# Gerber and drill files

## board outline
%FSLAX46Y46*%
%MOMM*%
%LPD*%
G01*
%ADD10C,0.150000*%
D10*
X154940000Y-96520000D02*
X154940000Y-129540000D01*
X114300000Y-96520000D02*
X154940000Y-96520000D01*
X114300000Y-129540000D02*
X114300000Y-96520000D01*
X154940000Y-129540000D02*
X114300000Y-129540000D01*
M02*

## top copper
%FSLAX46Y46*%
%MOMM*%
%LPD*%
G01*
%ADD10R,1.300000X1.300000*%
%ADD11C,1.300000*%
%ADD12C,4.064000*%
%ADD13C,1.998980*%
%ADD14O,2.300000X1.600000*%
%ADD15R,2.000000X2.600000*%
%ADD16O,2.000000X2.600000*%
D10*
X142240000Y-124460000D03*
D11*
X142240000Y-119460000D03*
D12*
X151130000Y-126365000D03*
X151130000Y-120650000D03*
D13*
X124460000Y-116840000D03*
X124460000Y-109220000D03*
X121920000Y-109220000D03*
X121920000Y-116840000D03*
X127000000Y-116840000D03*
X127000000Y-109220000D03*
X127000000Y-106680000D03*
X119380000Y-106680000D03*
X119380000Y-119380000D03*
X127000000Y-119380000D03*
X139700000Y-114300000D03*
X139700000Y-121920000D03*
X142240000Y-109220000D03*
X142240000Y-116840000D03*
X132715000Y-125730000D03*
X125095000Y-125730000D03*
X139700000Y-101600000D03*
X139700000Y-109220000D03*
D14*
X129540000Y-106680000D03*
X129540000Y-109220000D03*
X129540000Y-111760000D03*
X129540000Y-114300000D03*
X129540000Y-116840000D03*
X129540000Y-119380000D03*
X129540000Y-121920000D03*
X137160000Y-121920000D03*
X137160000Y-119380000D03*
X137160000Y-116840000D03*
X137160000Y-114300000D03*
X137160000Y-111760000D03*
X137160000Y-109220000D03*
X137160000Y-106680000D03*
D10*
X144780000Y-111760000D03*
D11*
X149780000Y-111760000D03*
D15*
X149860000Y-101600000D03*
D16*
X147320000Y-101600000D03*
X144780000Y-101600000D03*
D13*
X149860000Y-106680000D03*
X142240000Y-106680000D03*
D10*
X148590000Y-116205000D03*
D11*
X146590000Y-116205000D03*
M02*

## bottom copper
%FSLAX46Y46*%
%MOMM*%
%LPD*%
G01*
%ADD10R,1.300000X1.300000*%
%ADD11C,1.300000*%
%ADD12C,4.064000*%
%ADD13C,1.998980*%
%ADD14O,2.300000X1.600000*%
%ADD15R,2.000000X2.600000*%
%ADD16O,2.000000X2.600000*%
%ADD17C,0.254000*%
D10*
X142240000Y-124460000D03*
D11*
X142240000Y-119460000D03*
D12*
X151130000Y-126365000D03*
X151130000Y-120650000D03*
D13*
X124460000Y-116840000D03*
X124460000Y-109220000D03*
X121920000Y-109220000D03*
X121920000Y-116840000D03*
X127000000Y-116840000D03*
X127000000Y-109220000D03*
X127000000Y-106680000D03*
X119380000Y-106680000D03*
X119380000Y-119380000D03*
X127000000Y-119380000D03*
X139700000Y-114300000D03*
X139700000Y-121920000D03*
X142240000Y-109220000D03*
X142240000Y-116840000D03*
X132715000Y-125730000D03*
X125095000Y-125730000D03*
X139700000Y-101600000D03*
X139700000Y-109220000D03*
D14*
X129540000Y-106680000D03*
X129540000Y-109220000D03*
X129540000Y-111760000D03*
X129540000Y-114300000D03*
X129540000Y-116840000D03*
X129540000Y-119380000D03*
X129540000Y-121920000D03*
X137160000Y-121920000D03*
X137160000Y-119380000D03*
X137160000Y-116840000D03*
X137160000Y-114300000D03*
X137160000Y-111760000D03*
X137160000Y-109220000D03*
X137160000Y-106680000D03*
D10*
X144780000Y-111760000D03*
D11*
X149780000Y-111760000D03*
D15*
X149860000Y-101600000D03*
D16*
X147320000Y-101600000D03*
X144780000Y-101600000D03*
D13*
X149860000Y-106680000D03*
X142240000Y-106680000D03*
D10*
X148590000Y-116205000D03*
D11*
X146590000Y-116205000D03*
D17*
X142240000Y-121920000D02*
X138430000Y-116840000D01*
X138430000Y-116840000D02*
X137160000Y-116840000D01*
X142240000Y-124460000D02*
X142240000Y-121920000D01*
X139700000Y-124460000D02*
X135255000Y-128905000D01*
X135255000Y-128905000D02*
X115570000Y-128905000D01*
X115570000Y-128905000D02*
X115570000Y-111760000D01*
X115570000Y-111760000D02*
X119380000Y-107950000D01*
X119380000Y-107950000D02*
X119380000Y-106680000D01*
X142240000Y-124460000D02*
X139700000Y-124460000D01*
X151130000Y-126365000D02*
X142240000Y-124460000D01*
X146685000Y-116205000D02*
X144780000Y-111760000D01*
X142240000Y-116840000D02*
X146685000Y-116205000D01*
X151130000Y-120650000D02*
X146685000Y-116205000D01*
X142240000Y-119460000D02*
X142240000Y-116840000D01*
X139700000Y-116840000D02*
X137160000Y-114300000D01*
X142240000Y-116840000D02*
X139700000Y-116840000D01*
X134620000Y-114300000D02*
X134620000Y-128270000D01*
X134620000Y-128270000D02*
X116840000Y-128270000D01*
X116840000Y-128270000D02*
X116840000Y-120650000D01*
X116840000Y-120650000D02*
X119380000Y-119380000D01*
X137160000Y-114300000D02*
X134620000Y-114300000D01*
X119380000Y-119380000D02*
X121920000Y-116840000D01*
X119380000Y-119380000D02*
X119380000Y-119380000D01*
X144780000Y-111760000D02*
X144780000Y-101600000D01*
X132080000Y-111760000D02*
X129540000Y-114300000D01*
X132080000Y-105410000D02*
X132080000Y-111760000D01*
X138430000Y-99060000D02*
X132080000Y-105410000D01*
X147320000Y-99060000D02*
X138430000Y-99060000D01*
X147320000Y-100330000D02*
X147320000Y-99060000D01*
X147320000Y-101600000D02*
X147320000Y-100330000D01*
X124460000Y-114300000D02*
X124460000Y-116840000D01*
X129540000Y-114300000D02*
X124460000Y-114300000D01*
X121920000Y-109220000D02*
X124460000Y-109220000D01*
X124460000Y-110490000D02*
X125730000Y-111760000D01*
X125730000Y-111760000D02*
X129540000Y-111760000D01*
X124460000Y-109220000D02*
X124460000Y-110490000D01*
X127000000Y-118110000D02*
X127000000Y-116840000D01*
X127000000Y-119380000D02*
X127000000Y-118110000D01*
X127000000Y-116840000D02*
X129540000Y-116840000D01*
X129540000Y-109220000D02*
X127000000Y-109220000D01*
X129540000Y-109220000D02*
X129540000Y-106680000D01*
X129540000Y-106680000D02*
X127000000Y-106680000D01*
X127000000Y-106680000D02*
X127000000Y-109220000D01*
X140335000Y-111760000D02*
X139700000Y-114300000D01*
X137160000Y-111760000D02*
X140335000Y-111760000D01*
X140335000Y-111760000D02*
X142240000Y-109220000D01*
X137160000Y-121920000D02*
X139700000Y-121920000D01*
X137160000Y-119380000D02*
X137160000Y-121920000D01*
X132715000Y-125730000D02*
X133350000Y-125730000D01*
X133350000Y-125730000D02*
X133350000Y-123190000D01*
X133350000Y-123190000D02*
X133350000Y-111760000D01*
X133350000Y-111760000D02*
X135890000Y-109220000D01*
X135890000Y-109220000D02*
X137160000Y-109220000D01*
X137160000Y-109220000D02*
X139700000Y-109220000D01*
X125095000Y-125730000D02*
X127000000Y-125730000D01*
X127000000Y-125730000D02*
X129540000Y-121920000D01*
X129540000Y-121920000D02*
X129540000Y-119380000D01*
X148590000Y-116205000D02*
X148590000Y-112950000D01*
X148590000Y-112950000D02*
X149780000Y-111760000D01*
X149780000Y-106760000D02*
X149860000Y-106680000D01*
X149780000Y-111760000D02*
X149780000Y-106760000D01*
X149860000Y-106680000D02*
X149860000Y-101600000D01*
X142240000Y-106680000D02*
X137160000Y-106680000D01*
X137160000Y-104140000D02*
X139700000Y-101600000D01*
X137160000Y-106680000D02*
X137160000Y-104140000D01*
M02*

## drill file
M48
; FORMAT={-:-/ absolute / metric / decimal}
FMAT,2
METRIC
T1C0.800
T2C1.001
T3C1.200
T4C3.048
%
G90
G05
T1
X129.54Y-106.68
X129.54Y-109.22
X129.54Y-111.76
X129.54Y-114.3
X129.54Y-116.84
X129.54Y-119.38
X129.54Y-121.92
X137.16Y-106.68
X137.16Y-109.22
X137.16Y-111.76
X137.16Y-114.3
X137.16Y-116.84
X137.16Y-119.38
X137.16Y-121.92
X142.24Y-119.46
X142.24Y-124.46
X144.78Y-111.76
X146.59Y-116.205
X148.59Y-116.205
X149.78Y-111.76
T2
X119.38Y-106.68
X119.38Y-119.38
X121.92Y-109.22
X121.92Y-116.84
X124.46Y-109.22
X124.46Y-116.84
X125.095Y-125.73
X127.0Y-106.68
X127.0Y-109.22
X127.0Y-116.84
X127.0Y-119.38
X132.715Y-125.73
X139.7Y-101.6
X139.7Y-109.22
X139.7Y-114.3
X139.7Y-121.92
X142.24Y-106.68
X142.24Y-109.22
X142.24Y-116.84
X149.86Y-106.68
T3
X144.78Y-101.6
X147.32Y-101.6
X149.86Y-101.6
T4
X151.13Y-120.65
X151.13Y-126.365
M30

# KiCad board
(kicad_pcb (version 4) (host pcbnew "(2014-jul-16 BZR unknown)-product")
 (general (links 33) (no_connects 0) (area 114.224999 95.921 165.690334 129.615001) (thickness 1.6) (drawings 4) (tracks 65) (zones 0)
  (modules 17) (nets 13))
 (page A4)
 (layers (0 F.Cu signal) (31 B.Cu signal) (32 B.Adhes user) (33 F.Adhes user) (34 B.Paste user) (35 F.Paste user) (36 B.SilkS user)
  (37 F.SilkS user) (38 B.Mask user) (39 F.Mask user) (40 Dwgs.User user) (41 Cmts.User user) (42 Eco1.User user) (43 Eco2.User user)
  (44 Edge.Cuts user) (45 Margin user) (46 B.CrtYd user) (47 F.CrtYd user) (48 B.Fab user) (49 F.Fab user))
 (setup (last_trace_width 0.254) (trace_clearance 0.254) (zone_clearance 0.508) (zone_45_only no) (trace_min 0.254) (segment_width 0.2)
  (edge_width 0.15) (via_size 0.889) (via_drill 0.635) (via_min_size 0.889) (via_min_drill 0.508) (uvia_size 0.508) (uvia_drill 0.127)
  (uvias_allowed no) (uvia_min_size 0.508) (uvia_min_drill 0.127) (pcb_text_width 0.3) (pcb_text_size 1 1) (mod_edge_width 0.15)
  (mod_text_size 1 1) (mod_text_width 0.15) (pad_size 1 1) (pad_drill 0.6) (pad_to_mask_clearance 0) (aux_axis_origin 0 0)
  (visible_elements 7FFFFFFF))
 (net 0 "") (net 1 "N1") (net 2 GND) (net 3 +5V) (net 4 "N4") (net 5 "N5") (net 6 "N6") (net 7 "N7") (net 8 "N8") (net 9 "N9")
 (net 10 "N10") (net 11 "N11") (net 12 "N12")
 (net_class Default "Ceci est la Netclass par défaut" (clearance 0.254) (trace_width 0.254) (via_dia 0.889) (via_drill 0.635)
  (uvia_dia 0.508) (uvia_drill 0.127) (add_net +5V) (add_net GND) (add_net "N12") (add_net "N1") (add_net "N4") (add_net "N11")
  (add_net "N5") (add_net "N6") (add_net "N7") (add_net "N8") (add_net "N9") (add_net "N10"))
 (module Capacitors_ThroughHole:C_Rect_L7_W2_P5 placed (layer F.Cu) (at 142.24 124.46 90)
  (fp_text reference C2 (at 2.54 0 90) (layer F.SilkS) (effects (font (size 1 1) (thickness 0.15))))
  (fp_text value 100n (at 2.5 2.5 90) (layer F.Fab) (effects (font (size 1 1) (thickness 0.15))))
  (pad 1 thru_hole rect (at 0 0 90) (size 1.3 1.3) (drill 0.8) (layers *.Cu *.Mask F.SilkS) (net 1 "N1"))
  (pad 2 thru_hole circle (at 5 0 90) (size 1.3 1.3) (drill 0.8) (layers *.Cu *.Mask F.SilkS) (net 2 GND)))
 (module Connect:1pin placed (layer F.Cu) (at 151.13 126.365)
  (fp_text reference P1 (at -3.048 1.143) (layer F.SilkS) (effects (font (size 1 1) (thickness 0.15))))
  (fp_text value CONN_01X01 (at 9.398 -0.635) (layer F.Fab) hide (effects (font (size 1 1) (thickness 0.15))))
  (pad 1 thru_hole circle (at 0 0) (size 4.064 4.064) (drill 3.048) (layers *.Cu *.Mask F.SilkS) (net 1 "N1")))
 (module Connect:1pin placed (layer F.Cu) (at 151.13 120.65)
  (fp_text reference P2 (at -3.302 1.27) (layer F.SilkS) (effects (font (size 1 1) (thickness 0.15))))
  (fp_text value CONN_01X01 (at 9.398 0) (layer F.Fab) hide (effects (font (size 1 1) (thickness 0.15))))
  (pad 1 thru_hole circle (at 0 0) (size 4.064 4.064) (drill 3.048) (layers *.Cu *.Mask F.SilkS) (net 2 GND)))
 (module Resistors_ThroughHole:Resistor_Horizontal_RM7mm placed (layer F.Cu) (at 124.46 116.84 90)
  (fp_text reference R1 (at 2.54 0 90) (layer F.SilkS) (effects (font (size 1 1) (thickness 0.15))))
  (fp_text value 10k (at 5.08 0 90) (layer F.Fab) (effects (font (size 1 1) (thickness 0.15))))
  (pad 1 thru_hole circle (at 0 0 90) (size 1.99898 1.99898) (drill 1.00076) (layers *.Cu *.SilkS *.Mask) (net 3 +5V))
  (pad 2 thru_hole circle (at 7.62 0 90) (size 1.99898 1.99898) (drill 1.00076) (layers *.Cu *.SilkS *.Mask) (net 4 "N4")))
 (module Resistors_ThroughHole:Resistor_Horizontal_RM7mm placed (layer F.Cu) (at 121.92 109.22 270)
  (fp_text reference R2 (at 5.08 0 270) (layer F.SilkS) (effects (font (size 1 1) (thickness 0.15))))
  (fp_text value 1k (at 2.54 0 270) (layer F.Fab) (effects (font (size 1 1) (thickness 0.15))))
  (pad 1 thru_hole circle (at 0 0 270) (size 1.99898 1.99898) (drill 1.00076) (layers *.Cu *.SilkS *.Mask) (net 4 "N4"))
  (pad 2 thru_hole circle (at 7.62 0 270) (size 1.99898 1.99898) (drill 1.00076) (layers *.Cu *.SilkS *.Mask) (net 2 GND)))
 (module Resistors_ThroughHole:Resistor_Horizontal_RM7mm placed (layer F.Cu) (at 127 116.84 90)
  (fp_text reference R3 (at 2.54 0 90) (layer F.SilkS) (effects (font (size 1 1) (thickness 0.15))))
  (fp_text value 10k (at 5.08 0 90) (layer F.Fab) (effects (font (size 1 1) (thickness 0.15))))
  (pad 1 thru_hole circle (at 0 0 90) (size 1.99898 1.99898) (drill 1.00076) (layers *.Cu *.SilkS *.Mask) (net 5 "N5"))
  (pad 2 thru_hole circle (at 7.62 0 90) (size 1.99898 1.99898) (drill 1.00076) (layers *.Cu *.SilkS *.Mask) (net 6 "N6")))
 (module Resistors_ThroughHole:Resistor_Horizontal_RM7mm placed (layer F.Cu) (at 127 106.68 180)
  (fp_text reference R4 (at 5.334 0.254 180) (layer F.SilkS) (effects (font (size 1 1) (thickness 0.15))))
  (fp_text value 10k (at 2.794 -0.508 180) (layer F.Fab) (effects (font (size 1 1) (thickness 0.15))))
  (pad 1 thru_hole circle (at 0 0 180) (size 1.99898 1.99898) (drill 1.00076) (layers *.Cu *.SilkS *.Mask) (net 6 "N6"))
  (pad 2 thru_hole circle (at 7.62 0 180) (size 1.99898 1.99898) (drill 1.00076) (layers *.Cu *.SilkS *.Mask) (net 1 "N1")))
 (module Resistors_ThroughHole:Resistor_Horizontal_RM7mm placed (layer F.Cu) (at 119.38 119.38)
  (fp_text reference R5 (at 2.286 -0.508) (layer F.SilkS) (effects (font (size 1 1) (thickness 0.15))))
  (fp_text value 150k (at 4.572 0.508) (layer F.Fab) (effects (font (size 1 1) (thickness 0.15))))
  (pad 1 thru_hole circle (at 0 0) (size 1.99898 1.99898) (drill 1.00076) (layers *.Cu *.SilkS *.Mask) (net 2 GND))
  (pad 2 thru_hole circle (at 7.62 0) (size 1.99898 1.99898) (drill 1.00076) (layers *.Cu *.SilkS *.Mask) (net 5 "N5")))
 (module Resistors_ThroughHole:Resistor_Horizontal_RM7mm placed (layer F.Cu) (at 139.7 114.3 270)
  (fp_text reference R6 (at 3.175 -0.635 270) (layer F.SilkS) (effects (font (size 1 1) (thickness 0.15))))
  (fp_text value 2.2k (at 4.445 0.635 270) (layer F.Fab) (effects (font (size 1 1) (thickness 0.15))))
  (pad 1 thru_hole circle (at 0 0 270) (size 1.99898 1.99898) (drill 1.00076) (layers *.Cu *.SilkS *.Mask) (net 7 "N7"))
  (pad 2 thru_hole circle (at 7.62 0 270) (size 1.99898 1.99898) (drill 1.00076) (layers *.Cu *.SilkS *.Mask) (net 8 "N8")))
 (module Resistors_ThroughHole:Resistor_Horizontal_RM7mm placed (layer F.Cu) (at 142.24 109.22 270)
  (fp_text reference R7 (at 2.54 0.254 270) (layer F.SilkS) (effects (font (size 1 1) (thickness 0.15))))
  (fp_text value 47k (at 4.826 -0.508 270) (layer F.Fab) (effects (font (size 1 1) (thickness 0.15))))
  (pad 1 thru_hole circle (at 0 0 270) (size 1.99898 1.99898) (drill 1.00076) (layers *.Cu *.SilkS *.Mask) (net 7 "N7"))
  (pad 2 thru_hole circle (at 7.62 0 270) (size 1.99898 1.99898) (drill 1.00076) (layers *.Cu *.SilkS *.Mask) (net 2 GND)))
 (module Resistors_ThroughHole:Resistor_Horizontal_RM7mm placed (layer F.Cu) (at 132.715 125.73 180)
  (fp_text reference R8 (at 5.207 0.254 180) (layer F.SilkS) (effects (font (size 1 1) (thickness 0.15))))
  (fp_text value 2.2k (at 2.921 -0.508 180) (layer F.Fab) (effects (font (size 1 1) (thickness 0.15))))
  (pad 1 thru_hole circle (at 0 0 180) (size 1.99898 1.99898) (drill 1.00076) (layers *.Cu *.SilkS *.Mask) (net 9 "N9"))
  (pad 2 thru_hole circle (at 7.62 0 180) (size 1.99898 1.99898) (drill 1.00076) (layers *.Cu *.SilkS *.Mask) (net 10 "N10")))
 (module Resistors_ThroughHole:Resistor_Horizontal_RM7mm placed (layer F.Cu) (at 139.7 101.6 270)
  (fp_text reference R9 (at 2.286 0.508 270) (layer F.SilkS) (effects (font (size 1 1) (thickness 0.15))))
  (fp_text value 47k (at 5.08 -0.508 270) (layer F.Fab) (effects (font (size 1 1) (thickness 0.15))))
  (pad 1 thru_hole circle (at 0 0 270) (size 1.99898 1.99898) (drill 1.00076) (layers *.Cu *.SilkS *.Mask) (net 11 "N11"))
  (pad 2 thru_hole circle (at 7.62 0 270) (size 1.99898 1.99898) (drill 1.00076) (layers *.Cu *.SilkS *.Mask) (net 9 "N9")))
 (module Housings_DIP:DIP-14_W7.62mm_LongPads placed (layer F.Cu) (at 129.54 106.68)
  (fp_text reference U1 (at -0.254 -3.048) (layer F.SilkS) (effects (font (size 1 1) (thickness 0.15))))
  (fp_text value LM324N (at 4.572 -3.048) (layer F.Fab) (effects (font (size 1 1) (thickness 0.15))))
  (pad 1 thru_hole oval (at 0 0) (size 2.3 1.6) (drill 0.8) (layers *.Cu *.Mask F.SilkS) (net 6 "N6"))
  (pad 2 thru_hole oval (at 0 2.54) (size 2.3 1.6) (drill 0.8) (layers *.Cu *.Mask F.SilkS) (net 6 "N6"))
  (pad 3 thru_hole oval (at 0 5.08) (size 2.3 1.6) (drill 0.8) (layers *.Cu *.Mask F.SilkS) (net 4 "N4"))
  (pad 4 thru_hole oval (at 0 7.62) (size 2.3 1.6) (drill 0.8) (layers *.Cu *.Mask F.SilkS) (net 3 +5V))
  (pad 5 thru_hole oval (at 0 10.16) (size 2.3 1.6) (drill 0.8) (layers *.Cu *.Mask F.SilkS) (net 5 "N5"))
  (pad 6 thru_hole oval (at 0 12.7) (size 2.3 1.6) (drill 0.8) (layers *.Cu *.Mask F.SilkS) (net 10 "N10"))
  (pad 7 thru_hole oval (at 0 15.24) (size 2.3 1.6) (drill 0.8) (layers *.Cu *.Mask F.SilkS) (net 10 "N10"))
  (pad 8 thru_hole oval (at 7.62 15.24) (size 2.3 1.6) (drill 0.8) (layers *.Cu *.Mask F.SilkS) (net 8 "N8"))
  (pad 9 thru_hole oval (at 7.62 12.7) (size 2.3 1.6) (drill 0.8) (layers *.Cu *.Mask F.SilkS) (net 8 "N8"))
  (pad 10 thru_hole oval (at 7.62 10.16) (size 2.3 1.6) (drill 0.8) (layers *.Cu *.Mask F.SilkS) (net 1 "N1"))
  (pad 11 thru_hole oval (at 7.62 7.62) (size 2.3 1.6) (drill 0.8) (layers *.Cu *.Mask F.SilkS) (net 2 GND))
  (pad 12 thru_hole oval (at 7.62 5.08) (size 2.3 1.6) (drill 0.8) (layers *.Cu *.Mask F.SilkS) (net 7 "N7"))
  (pad 13 thru_hole oval (at 7.62 2.54) (size 2.3 1.6) (drill 0.8) (layers *.Cu *.Mask F.SilkS) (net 9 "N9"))
  (pad 14 thru_hole oval (at 7.62 0) (size 2.3 1.6) (drill 0.8) (layers *.Cu *.Mask F.SilkS) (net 11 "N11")))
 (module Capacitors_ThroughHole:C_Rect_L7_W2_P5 (layer F.Cu) (at 144.78 111.76)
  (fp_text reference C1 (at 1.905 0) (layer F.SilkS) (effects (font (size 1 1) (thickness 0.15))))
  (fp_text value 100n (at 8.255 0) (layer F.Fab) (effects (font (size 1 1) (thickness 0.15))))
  (pad 1 thru_hole rect (at 0 0) (size 1.3 1.3) (drill 0.8) (layers *.Cu *.Mask F.SilkS) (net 2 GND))
  (pad 2 thru_hole circle (at 5 0) (size 1.3 1.3) (drill 0.8) (layers *.Cu *.Mask F.SilkS) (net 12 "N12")))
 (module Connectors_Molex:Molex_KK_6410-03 (layer F.Cu) (at 149.86 101.6 180)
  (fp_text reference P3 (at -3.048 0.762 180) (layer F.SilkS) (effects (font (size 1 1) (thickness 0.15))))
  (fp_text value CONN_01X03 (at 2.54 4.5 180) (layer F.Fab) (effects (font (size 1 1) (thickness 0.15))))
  (pad 1 thru_hole rect (at 0 0 180) (size 2 2.6) (drill 1.2) (layers *.Cu *.Mask F.SilkS) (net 12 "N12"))
  (pad 2 thru_hole oval (at 2.54 0 180) (size 2 2.6) (drill 1.2) (layers *.Cu *.Mask F.SilkS) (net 3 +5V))
  (pad 3 thru_hole oval (at 5.08 0 180) (size 2 2.6) (drill 1.2) (layers *.Cu *.Mask F.SilkS) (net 2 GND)))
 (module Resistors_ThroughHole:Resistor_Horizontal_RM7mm (layer F.Cu) (at 149.86 106.68 180)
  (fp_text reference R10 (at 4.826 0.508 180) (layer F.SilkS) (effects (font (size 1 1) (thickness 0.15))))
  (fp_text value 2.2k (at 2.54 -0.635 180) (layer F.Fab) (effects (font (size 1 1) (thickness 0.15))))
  (pad 1 thru_hole circle (at 0 0 180) (size 1.99898 1.99898) (drill 1.00076) (layers *.Cu *.SilkS *.Mask) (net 12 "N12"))
  (pad 2 thru_hole circle (at 7.62 0 180) (size 1.99898 1.99898) (drill 1.00076) (layers *.Cu *.SilkS *.Mask) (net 11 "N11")))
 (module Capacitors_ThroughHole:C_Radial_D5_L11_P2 (layer F.Cu) (at 148.59 116.205 180)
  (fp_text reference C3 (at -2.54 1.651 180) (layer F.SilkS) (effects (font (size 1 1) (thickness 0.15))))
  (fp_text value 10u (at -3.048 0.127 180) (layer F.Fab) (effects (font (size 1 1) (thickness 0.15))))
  (pad 1 thru_hole rect (at 0 0 180) (size 1.3 1.3) (drill 0.8) (layers *.Cu *.Mask F.SilkS) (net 12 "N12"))
  (pad 2 thru_hole circle (at 2 0 180) (size 1.3 1.3) (drill 0.8) (layers *.Cu *.Mask F.SilkS) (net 2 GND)))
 (gr_line (start 154.94 96.52) (end 154.94 129.54) (angle 90) (layer Edge.Cuts) (width 0.15))
 (gr_line (start 114.3 96.52) (end 154.94 96.52) (angle 90) (layer Edge.Cuts) (width 0.15))
 (gr_line (start 114.3 129.54) (end 114.3 96.52) (angle 90) (layer Edge.Cuts) (width 0.15))
 (gr_line (start 154.94 129.54) (end 114.3 129.54) (angle 90) (layer Edge.Cuts) (width 0.15))
 (segment (start 142.24 121.92) (end 138.43 116.84) (width 0.254) (layer B.Cu) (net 1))
 (segment (start 138.43 116.84) (end 137.16 116.84) (width 0.254) (layer B.Cu) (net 1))
 (segment (start 142.24 124.46) (end 142.24 121.92) (width 0.254) (layer B.Cu) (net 1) (status 10))
 (segment (start 139.7 124.46) (end 135.255 128.905) (width 0.254) (layer B.Cu) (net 1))
 (segment (start 135.255 128.905) (end 115.57 128.905) (width 0.254) (layer B.Cu) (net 1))
 (segment (start 115.57 128.905) (end 115.57 111.76) (width 0.254) (layer B.Cu) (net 1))
 (segment (start 115.57 111.76) (end 119.38 107.95) (width 0.254) (layer B.Cu) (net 1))
 (segment (start 119.38 107.95) (end 119.38 106.68) (width 0.254) (layer B.Cu) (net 1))
 (segment (start 142.24 124.46) (end 139.7 124.46) (width 0.254) (layer B.Cu) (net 1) (status 10))
 (segment (start 151.13 126.365) (end 142.24 124.46) (width 0.254) (layer B.Cu) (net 1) (status 10))
 (segment (start 146.685 116.205) (end 144.78 111.76) (width 0.254) (layer B.Cu) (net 2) (status 800020))
 (segment (start 142.24 116.84) (end 146.685 116.205) (width 0.254) (layer B.Cu) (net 2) (status 400010))
 (segment (start 151.13 120.65) (end 146.685 116.205) (width 0.254) (layer B.Cu) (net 2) (status 400010))
 (segment (start 142.24 119.46) (end 142.24 116.84) (width 0.254) (layer B.Cu) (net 2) (status 10))
 (segment (start 139.7 116.84) (end 137.16 114.3) (width 0.254) (layer B.Cu) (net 2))
 (segment (start 142.24 116.84) (end 139.7 116.84) (width 0.254) (layer B.Cu) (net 2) (status 10))
 (segment (start 134.62 114.3) (end 134.62 128.27) (width 0.254) (layer B.Cu) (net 2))
 (segment (start 134.62 128.27) (end 116.84 128.27) (width 0.254) (layer B.Cu) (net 2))
 (segment (start 116.84 128.27) (end 116.84 120.65) (width 0.254) (layer B.Cu) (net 2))
 (segment (start 116.84 120.65) (end 119.38 119.38) (width 0.254) (layer B.Cu) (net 2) (status 20))
 (segment (start 137.16 114.3) (end 134.62 114.3) (width 0.254) (layer B.Cu) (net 2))
 (segment (start 119.38 119.38) (end 121.92 116.84) (width 0.254) (layer B.Cu) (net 2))
 (segment (start 119.38 119.38) (end 119.38 119.38) (width 0.254) (layer B.Cu) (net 2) (status 10))
 (segment (start 144.78 111.76) (end 144.78 101.6) (width 0.254) (layer B.Cu) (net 2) (status 20))
 (segment (start 132.08 111.76) (end 129.54 114.3) (width 0.254) (layer B.Cu) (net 3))
 (segment (start 132.08 105.41) (end 132.08 111.76) (width 0.254) (layer B.Cu) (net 3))
 (segment (start 138.43 99.06) (end 132.08 105.41) (width 0.254) (layer B.Cu) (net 3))
 (segment (start 147.32 99.06) (end 138.43 99.06) (width 0.254) (layer B.Cu) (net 3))
 (segment (start 147.32 100.33) (end 147.32 99.06) (width 0.254) (layer B.Cu) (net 3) (status 10))
 (segment (start 147.32 101.6) (end 147.32 100.33) (width 0.254) (layer B.Cu) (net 3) (status 30))
 (segment (start 124.46 114.3) (end 124.46 116.84) (width 0.254) (layer B.Cu) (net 3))
 (segment (start 129.54 114.3) (end 124.46 114.3) (width 0.254) (layer B.Cu) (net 3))
 (segment (start 121.92 109.22) (end 124.46 109.22) (width 0.254) (layer B.Cu) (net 4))
 (segment (start 124.46 110.49) (end 125.73 111.76) (width 0.254) (layer B.Cu) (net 4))
 (segment (start 125.73 111.76) (end 129.54 111.76) (width 0.254) (layer B.Cu) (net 4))
 (segment (start 124.46 109.22) (end 124.46 110.49) (width 0.254) (layer B.Cu) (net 4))
 (segment (start 127 118.11) (end 127 116.84) (width 0.254) (layer B.Cu) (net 5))
 (segment (start 127 119.38) (end 127 118.11) (width 0.254) (layer B.Cu) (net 5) (status 10))
 (segment (start 127 116.84) (end 129.54 116.84) (width 0.254) (layer B.Cu) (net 5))
 (segment (start 129.54 109.22) (end 127 109.22) (width 0.254) (layer B.Cu) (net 6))
 (segment (start 129.54 109.22) (end 129.54 106.68) (width 0.254) (layer B.Cu) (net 6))
 (segment (start 129.54 106.68) (end 127 106.68) (width 0.254) (layer B.Cu) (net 6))
 (segment (start 127 106.68) (end 127 109.22) (width 0.254) (layer B.Cu) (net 6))
 (segment (start 140.335 111.76) (end 139.7 114.3) (width 0.254) (layer B.Cu) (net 7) (status 20))
 (segment (start 137.16 111.76) (end 140.335 111.76) (width 0.254) (layer B.Cu) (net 7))
 (segment (start 140.335 111.76) (end 142.24 109.22) (width 0.254) (layer B.Cu) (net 7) (status 20))
 (segment (start 137.16 121.92) (end 139.7 121.92) (width 0.254) (layer B.Cu) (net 8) (status 20))
 (segment (start 137.16 119.38) (end 137.16 121.92) (width 0.254) (layer B.Cu) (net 8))
 (segment (start 132.715 125.73) (end 133.35 125.73) (width 0.254) (layer B.Cu) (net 9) (status 10))
 (segment (start 133.35 125.73) (end 133.35 123.19) (width 0.254) (layer B.Cu) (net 9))
 (segment (start 133.35 123.19) (end 133.35 111.76) (width 0.254) (layer B.Cu) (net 9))
 (segment (start 133.35 111.76) (end 135.89 109.22) (width 0.254) (layer B.Cu) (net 9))
 (segment (start 135.89 109.22) (end 137.16 109.22) (width 0.254) (layer B.Cu) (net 9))
 (segment (start 137.16 109.22) (end 139.7 109.22) (width 0.254) (layer B.Cu) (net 9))
 (segment (start 125.095 125.73) (end 127 125.73) (width 0.254) (layer B.Cu) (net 10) (status 10))
 (segment (start 127 125.73) (end 129.54 121.92) (width 0.254) (layer B.Cu) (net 10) (status 10))
 (segment (start 129.54 121.92) (end 129.54 119.38) (width 0.254) (layer B.Cu) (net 10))
 (segment (start 148.59 116.205) (end 148.59 112.95) (width 0.254) (layer B.Cu) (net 12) (status 400000))
 (segment (start 148.59 112.95) (end 149.78 111.76) (width 0.254) (layer B.Cu) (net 12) (status 800000))
 (segment (start 149.78 106.76) (end 149.86 106.68) (width 0.254) (layer B.Cu) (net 12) (status 30))
 (segment (start 149.78 111.76) (end 149.78 106.76) (width 0.254) (layer B.Cu) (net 12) (status 20))
 (segment (start 149.86 106.68) (end 149.86 101.6) (width 0.254) (layer B.Cu) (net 12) (status 20))
 (segment (start 142.24 106.68) (end 137.16 106.68) (width 0.254) (layer B.Cu) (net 11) (status 10))
 (segment (start 137.16 104.14) (end 139.7 101.6) (width 0.254) (layer B.Cu) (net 11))
 (segment (start 137.16 106.68) (end 137.16 104.14) (width 0.254) (layer B.Cu) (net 11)))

